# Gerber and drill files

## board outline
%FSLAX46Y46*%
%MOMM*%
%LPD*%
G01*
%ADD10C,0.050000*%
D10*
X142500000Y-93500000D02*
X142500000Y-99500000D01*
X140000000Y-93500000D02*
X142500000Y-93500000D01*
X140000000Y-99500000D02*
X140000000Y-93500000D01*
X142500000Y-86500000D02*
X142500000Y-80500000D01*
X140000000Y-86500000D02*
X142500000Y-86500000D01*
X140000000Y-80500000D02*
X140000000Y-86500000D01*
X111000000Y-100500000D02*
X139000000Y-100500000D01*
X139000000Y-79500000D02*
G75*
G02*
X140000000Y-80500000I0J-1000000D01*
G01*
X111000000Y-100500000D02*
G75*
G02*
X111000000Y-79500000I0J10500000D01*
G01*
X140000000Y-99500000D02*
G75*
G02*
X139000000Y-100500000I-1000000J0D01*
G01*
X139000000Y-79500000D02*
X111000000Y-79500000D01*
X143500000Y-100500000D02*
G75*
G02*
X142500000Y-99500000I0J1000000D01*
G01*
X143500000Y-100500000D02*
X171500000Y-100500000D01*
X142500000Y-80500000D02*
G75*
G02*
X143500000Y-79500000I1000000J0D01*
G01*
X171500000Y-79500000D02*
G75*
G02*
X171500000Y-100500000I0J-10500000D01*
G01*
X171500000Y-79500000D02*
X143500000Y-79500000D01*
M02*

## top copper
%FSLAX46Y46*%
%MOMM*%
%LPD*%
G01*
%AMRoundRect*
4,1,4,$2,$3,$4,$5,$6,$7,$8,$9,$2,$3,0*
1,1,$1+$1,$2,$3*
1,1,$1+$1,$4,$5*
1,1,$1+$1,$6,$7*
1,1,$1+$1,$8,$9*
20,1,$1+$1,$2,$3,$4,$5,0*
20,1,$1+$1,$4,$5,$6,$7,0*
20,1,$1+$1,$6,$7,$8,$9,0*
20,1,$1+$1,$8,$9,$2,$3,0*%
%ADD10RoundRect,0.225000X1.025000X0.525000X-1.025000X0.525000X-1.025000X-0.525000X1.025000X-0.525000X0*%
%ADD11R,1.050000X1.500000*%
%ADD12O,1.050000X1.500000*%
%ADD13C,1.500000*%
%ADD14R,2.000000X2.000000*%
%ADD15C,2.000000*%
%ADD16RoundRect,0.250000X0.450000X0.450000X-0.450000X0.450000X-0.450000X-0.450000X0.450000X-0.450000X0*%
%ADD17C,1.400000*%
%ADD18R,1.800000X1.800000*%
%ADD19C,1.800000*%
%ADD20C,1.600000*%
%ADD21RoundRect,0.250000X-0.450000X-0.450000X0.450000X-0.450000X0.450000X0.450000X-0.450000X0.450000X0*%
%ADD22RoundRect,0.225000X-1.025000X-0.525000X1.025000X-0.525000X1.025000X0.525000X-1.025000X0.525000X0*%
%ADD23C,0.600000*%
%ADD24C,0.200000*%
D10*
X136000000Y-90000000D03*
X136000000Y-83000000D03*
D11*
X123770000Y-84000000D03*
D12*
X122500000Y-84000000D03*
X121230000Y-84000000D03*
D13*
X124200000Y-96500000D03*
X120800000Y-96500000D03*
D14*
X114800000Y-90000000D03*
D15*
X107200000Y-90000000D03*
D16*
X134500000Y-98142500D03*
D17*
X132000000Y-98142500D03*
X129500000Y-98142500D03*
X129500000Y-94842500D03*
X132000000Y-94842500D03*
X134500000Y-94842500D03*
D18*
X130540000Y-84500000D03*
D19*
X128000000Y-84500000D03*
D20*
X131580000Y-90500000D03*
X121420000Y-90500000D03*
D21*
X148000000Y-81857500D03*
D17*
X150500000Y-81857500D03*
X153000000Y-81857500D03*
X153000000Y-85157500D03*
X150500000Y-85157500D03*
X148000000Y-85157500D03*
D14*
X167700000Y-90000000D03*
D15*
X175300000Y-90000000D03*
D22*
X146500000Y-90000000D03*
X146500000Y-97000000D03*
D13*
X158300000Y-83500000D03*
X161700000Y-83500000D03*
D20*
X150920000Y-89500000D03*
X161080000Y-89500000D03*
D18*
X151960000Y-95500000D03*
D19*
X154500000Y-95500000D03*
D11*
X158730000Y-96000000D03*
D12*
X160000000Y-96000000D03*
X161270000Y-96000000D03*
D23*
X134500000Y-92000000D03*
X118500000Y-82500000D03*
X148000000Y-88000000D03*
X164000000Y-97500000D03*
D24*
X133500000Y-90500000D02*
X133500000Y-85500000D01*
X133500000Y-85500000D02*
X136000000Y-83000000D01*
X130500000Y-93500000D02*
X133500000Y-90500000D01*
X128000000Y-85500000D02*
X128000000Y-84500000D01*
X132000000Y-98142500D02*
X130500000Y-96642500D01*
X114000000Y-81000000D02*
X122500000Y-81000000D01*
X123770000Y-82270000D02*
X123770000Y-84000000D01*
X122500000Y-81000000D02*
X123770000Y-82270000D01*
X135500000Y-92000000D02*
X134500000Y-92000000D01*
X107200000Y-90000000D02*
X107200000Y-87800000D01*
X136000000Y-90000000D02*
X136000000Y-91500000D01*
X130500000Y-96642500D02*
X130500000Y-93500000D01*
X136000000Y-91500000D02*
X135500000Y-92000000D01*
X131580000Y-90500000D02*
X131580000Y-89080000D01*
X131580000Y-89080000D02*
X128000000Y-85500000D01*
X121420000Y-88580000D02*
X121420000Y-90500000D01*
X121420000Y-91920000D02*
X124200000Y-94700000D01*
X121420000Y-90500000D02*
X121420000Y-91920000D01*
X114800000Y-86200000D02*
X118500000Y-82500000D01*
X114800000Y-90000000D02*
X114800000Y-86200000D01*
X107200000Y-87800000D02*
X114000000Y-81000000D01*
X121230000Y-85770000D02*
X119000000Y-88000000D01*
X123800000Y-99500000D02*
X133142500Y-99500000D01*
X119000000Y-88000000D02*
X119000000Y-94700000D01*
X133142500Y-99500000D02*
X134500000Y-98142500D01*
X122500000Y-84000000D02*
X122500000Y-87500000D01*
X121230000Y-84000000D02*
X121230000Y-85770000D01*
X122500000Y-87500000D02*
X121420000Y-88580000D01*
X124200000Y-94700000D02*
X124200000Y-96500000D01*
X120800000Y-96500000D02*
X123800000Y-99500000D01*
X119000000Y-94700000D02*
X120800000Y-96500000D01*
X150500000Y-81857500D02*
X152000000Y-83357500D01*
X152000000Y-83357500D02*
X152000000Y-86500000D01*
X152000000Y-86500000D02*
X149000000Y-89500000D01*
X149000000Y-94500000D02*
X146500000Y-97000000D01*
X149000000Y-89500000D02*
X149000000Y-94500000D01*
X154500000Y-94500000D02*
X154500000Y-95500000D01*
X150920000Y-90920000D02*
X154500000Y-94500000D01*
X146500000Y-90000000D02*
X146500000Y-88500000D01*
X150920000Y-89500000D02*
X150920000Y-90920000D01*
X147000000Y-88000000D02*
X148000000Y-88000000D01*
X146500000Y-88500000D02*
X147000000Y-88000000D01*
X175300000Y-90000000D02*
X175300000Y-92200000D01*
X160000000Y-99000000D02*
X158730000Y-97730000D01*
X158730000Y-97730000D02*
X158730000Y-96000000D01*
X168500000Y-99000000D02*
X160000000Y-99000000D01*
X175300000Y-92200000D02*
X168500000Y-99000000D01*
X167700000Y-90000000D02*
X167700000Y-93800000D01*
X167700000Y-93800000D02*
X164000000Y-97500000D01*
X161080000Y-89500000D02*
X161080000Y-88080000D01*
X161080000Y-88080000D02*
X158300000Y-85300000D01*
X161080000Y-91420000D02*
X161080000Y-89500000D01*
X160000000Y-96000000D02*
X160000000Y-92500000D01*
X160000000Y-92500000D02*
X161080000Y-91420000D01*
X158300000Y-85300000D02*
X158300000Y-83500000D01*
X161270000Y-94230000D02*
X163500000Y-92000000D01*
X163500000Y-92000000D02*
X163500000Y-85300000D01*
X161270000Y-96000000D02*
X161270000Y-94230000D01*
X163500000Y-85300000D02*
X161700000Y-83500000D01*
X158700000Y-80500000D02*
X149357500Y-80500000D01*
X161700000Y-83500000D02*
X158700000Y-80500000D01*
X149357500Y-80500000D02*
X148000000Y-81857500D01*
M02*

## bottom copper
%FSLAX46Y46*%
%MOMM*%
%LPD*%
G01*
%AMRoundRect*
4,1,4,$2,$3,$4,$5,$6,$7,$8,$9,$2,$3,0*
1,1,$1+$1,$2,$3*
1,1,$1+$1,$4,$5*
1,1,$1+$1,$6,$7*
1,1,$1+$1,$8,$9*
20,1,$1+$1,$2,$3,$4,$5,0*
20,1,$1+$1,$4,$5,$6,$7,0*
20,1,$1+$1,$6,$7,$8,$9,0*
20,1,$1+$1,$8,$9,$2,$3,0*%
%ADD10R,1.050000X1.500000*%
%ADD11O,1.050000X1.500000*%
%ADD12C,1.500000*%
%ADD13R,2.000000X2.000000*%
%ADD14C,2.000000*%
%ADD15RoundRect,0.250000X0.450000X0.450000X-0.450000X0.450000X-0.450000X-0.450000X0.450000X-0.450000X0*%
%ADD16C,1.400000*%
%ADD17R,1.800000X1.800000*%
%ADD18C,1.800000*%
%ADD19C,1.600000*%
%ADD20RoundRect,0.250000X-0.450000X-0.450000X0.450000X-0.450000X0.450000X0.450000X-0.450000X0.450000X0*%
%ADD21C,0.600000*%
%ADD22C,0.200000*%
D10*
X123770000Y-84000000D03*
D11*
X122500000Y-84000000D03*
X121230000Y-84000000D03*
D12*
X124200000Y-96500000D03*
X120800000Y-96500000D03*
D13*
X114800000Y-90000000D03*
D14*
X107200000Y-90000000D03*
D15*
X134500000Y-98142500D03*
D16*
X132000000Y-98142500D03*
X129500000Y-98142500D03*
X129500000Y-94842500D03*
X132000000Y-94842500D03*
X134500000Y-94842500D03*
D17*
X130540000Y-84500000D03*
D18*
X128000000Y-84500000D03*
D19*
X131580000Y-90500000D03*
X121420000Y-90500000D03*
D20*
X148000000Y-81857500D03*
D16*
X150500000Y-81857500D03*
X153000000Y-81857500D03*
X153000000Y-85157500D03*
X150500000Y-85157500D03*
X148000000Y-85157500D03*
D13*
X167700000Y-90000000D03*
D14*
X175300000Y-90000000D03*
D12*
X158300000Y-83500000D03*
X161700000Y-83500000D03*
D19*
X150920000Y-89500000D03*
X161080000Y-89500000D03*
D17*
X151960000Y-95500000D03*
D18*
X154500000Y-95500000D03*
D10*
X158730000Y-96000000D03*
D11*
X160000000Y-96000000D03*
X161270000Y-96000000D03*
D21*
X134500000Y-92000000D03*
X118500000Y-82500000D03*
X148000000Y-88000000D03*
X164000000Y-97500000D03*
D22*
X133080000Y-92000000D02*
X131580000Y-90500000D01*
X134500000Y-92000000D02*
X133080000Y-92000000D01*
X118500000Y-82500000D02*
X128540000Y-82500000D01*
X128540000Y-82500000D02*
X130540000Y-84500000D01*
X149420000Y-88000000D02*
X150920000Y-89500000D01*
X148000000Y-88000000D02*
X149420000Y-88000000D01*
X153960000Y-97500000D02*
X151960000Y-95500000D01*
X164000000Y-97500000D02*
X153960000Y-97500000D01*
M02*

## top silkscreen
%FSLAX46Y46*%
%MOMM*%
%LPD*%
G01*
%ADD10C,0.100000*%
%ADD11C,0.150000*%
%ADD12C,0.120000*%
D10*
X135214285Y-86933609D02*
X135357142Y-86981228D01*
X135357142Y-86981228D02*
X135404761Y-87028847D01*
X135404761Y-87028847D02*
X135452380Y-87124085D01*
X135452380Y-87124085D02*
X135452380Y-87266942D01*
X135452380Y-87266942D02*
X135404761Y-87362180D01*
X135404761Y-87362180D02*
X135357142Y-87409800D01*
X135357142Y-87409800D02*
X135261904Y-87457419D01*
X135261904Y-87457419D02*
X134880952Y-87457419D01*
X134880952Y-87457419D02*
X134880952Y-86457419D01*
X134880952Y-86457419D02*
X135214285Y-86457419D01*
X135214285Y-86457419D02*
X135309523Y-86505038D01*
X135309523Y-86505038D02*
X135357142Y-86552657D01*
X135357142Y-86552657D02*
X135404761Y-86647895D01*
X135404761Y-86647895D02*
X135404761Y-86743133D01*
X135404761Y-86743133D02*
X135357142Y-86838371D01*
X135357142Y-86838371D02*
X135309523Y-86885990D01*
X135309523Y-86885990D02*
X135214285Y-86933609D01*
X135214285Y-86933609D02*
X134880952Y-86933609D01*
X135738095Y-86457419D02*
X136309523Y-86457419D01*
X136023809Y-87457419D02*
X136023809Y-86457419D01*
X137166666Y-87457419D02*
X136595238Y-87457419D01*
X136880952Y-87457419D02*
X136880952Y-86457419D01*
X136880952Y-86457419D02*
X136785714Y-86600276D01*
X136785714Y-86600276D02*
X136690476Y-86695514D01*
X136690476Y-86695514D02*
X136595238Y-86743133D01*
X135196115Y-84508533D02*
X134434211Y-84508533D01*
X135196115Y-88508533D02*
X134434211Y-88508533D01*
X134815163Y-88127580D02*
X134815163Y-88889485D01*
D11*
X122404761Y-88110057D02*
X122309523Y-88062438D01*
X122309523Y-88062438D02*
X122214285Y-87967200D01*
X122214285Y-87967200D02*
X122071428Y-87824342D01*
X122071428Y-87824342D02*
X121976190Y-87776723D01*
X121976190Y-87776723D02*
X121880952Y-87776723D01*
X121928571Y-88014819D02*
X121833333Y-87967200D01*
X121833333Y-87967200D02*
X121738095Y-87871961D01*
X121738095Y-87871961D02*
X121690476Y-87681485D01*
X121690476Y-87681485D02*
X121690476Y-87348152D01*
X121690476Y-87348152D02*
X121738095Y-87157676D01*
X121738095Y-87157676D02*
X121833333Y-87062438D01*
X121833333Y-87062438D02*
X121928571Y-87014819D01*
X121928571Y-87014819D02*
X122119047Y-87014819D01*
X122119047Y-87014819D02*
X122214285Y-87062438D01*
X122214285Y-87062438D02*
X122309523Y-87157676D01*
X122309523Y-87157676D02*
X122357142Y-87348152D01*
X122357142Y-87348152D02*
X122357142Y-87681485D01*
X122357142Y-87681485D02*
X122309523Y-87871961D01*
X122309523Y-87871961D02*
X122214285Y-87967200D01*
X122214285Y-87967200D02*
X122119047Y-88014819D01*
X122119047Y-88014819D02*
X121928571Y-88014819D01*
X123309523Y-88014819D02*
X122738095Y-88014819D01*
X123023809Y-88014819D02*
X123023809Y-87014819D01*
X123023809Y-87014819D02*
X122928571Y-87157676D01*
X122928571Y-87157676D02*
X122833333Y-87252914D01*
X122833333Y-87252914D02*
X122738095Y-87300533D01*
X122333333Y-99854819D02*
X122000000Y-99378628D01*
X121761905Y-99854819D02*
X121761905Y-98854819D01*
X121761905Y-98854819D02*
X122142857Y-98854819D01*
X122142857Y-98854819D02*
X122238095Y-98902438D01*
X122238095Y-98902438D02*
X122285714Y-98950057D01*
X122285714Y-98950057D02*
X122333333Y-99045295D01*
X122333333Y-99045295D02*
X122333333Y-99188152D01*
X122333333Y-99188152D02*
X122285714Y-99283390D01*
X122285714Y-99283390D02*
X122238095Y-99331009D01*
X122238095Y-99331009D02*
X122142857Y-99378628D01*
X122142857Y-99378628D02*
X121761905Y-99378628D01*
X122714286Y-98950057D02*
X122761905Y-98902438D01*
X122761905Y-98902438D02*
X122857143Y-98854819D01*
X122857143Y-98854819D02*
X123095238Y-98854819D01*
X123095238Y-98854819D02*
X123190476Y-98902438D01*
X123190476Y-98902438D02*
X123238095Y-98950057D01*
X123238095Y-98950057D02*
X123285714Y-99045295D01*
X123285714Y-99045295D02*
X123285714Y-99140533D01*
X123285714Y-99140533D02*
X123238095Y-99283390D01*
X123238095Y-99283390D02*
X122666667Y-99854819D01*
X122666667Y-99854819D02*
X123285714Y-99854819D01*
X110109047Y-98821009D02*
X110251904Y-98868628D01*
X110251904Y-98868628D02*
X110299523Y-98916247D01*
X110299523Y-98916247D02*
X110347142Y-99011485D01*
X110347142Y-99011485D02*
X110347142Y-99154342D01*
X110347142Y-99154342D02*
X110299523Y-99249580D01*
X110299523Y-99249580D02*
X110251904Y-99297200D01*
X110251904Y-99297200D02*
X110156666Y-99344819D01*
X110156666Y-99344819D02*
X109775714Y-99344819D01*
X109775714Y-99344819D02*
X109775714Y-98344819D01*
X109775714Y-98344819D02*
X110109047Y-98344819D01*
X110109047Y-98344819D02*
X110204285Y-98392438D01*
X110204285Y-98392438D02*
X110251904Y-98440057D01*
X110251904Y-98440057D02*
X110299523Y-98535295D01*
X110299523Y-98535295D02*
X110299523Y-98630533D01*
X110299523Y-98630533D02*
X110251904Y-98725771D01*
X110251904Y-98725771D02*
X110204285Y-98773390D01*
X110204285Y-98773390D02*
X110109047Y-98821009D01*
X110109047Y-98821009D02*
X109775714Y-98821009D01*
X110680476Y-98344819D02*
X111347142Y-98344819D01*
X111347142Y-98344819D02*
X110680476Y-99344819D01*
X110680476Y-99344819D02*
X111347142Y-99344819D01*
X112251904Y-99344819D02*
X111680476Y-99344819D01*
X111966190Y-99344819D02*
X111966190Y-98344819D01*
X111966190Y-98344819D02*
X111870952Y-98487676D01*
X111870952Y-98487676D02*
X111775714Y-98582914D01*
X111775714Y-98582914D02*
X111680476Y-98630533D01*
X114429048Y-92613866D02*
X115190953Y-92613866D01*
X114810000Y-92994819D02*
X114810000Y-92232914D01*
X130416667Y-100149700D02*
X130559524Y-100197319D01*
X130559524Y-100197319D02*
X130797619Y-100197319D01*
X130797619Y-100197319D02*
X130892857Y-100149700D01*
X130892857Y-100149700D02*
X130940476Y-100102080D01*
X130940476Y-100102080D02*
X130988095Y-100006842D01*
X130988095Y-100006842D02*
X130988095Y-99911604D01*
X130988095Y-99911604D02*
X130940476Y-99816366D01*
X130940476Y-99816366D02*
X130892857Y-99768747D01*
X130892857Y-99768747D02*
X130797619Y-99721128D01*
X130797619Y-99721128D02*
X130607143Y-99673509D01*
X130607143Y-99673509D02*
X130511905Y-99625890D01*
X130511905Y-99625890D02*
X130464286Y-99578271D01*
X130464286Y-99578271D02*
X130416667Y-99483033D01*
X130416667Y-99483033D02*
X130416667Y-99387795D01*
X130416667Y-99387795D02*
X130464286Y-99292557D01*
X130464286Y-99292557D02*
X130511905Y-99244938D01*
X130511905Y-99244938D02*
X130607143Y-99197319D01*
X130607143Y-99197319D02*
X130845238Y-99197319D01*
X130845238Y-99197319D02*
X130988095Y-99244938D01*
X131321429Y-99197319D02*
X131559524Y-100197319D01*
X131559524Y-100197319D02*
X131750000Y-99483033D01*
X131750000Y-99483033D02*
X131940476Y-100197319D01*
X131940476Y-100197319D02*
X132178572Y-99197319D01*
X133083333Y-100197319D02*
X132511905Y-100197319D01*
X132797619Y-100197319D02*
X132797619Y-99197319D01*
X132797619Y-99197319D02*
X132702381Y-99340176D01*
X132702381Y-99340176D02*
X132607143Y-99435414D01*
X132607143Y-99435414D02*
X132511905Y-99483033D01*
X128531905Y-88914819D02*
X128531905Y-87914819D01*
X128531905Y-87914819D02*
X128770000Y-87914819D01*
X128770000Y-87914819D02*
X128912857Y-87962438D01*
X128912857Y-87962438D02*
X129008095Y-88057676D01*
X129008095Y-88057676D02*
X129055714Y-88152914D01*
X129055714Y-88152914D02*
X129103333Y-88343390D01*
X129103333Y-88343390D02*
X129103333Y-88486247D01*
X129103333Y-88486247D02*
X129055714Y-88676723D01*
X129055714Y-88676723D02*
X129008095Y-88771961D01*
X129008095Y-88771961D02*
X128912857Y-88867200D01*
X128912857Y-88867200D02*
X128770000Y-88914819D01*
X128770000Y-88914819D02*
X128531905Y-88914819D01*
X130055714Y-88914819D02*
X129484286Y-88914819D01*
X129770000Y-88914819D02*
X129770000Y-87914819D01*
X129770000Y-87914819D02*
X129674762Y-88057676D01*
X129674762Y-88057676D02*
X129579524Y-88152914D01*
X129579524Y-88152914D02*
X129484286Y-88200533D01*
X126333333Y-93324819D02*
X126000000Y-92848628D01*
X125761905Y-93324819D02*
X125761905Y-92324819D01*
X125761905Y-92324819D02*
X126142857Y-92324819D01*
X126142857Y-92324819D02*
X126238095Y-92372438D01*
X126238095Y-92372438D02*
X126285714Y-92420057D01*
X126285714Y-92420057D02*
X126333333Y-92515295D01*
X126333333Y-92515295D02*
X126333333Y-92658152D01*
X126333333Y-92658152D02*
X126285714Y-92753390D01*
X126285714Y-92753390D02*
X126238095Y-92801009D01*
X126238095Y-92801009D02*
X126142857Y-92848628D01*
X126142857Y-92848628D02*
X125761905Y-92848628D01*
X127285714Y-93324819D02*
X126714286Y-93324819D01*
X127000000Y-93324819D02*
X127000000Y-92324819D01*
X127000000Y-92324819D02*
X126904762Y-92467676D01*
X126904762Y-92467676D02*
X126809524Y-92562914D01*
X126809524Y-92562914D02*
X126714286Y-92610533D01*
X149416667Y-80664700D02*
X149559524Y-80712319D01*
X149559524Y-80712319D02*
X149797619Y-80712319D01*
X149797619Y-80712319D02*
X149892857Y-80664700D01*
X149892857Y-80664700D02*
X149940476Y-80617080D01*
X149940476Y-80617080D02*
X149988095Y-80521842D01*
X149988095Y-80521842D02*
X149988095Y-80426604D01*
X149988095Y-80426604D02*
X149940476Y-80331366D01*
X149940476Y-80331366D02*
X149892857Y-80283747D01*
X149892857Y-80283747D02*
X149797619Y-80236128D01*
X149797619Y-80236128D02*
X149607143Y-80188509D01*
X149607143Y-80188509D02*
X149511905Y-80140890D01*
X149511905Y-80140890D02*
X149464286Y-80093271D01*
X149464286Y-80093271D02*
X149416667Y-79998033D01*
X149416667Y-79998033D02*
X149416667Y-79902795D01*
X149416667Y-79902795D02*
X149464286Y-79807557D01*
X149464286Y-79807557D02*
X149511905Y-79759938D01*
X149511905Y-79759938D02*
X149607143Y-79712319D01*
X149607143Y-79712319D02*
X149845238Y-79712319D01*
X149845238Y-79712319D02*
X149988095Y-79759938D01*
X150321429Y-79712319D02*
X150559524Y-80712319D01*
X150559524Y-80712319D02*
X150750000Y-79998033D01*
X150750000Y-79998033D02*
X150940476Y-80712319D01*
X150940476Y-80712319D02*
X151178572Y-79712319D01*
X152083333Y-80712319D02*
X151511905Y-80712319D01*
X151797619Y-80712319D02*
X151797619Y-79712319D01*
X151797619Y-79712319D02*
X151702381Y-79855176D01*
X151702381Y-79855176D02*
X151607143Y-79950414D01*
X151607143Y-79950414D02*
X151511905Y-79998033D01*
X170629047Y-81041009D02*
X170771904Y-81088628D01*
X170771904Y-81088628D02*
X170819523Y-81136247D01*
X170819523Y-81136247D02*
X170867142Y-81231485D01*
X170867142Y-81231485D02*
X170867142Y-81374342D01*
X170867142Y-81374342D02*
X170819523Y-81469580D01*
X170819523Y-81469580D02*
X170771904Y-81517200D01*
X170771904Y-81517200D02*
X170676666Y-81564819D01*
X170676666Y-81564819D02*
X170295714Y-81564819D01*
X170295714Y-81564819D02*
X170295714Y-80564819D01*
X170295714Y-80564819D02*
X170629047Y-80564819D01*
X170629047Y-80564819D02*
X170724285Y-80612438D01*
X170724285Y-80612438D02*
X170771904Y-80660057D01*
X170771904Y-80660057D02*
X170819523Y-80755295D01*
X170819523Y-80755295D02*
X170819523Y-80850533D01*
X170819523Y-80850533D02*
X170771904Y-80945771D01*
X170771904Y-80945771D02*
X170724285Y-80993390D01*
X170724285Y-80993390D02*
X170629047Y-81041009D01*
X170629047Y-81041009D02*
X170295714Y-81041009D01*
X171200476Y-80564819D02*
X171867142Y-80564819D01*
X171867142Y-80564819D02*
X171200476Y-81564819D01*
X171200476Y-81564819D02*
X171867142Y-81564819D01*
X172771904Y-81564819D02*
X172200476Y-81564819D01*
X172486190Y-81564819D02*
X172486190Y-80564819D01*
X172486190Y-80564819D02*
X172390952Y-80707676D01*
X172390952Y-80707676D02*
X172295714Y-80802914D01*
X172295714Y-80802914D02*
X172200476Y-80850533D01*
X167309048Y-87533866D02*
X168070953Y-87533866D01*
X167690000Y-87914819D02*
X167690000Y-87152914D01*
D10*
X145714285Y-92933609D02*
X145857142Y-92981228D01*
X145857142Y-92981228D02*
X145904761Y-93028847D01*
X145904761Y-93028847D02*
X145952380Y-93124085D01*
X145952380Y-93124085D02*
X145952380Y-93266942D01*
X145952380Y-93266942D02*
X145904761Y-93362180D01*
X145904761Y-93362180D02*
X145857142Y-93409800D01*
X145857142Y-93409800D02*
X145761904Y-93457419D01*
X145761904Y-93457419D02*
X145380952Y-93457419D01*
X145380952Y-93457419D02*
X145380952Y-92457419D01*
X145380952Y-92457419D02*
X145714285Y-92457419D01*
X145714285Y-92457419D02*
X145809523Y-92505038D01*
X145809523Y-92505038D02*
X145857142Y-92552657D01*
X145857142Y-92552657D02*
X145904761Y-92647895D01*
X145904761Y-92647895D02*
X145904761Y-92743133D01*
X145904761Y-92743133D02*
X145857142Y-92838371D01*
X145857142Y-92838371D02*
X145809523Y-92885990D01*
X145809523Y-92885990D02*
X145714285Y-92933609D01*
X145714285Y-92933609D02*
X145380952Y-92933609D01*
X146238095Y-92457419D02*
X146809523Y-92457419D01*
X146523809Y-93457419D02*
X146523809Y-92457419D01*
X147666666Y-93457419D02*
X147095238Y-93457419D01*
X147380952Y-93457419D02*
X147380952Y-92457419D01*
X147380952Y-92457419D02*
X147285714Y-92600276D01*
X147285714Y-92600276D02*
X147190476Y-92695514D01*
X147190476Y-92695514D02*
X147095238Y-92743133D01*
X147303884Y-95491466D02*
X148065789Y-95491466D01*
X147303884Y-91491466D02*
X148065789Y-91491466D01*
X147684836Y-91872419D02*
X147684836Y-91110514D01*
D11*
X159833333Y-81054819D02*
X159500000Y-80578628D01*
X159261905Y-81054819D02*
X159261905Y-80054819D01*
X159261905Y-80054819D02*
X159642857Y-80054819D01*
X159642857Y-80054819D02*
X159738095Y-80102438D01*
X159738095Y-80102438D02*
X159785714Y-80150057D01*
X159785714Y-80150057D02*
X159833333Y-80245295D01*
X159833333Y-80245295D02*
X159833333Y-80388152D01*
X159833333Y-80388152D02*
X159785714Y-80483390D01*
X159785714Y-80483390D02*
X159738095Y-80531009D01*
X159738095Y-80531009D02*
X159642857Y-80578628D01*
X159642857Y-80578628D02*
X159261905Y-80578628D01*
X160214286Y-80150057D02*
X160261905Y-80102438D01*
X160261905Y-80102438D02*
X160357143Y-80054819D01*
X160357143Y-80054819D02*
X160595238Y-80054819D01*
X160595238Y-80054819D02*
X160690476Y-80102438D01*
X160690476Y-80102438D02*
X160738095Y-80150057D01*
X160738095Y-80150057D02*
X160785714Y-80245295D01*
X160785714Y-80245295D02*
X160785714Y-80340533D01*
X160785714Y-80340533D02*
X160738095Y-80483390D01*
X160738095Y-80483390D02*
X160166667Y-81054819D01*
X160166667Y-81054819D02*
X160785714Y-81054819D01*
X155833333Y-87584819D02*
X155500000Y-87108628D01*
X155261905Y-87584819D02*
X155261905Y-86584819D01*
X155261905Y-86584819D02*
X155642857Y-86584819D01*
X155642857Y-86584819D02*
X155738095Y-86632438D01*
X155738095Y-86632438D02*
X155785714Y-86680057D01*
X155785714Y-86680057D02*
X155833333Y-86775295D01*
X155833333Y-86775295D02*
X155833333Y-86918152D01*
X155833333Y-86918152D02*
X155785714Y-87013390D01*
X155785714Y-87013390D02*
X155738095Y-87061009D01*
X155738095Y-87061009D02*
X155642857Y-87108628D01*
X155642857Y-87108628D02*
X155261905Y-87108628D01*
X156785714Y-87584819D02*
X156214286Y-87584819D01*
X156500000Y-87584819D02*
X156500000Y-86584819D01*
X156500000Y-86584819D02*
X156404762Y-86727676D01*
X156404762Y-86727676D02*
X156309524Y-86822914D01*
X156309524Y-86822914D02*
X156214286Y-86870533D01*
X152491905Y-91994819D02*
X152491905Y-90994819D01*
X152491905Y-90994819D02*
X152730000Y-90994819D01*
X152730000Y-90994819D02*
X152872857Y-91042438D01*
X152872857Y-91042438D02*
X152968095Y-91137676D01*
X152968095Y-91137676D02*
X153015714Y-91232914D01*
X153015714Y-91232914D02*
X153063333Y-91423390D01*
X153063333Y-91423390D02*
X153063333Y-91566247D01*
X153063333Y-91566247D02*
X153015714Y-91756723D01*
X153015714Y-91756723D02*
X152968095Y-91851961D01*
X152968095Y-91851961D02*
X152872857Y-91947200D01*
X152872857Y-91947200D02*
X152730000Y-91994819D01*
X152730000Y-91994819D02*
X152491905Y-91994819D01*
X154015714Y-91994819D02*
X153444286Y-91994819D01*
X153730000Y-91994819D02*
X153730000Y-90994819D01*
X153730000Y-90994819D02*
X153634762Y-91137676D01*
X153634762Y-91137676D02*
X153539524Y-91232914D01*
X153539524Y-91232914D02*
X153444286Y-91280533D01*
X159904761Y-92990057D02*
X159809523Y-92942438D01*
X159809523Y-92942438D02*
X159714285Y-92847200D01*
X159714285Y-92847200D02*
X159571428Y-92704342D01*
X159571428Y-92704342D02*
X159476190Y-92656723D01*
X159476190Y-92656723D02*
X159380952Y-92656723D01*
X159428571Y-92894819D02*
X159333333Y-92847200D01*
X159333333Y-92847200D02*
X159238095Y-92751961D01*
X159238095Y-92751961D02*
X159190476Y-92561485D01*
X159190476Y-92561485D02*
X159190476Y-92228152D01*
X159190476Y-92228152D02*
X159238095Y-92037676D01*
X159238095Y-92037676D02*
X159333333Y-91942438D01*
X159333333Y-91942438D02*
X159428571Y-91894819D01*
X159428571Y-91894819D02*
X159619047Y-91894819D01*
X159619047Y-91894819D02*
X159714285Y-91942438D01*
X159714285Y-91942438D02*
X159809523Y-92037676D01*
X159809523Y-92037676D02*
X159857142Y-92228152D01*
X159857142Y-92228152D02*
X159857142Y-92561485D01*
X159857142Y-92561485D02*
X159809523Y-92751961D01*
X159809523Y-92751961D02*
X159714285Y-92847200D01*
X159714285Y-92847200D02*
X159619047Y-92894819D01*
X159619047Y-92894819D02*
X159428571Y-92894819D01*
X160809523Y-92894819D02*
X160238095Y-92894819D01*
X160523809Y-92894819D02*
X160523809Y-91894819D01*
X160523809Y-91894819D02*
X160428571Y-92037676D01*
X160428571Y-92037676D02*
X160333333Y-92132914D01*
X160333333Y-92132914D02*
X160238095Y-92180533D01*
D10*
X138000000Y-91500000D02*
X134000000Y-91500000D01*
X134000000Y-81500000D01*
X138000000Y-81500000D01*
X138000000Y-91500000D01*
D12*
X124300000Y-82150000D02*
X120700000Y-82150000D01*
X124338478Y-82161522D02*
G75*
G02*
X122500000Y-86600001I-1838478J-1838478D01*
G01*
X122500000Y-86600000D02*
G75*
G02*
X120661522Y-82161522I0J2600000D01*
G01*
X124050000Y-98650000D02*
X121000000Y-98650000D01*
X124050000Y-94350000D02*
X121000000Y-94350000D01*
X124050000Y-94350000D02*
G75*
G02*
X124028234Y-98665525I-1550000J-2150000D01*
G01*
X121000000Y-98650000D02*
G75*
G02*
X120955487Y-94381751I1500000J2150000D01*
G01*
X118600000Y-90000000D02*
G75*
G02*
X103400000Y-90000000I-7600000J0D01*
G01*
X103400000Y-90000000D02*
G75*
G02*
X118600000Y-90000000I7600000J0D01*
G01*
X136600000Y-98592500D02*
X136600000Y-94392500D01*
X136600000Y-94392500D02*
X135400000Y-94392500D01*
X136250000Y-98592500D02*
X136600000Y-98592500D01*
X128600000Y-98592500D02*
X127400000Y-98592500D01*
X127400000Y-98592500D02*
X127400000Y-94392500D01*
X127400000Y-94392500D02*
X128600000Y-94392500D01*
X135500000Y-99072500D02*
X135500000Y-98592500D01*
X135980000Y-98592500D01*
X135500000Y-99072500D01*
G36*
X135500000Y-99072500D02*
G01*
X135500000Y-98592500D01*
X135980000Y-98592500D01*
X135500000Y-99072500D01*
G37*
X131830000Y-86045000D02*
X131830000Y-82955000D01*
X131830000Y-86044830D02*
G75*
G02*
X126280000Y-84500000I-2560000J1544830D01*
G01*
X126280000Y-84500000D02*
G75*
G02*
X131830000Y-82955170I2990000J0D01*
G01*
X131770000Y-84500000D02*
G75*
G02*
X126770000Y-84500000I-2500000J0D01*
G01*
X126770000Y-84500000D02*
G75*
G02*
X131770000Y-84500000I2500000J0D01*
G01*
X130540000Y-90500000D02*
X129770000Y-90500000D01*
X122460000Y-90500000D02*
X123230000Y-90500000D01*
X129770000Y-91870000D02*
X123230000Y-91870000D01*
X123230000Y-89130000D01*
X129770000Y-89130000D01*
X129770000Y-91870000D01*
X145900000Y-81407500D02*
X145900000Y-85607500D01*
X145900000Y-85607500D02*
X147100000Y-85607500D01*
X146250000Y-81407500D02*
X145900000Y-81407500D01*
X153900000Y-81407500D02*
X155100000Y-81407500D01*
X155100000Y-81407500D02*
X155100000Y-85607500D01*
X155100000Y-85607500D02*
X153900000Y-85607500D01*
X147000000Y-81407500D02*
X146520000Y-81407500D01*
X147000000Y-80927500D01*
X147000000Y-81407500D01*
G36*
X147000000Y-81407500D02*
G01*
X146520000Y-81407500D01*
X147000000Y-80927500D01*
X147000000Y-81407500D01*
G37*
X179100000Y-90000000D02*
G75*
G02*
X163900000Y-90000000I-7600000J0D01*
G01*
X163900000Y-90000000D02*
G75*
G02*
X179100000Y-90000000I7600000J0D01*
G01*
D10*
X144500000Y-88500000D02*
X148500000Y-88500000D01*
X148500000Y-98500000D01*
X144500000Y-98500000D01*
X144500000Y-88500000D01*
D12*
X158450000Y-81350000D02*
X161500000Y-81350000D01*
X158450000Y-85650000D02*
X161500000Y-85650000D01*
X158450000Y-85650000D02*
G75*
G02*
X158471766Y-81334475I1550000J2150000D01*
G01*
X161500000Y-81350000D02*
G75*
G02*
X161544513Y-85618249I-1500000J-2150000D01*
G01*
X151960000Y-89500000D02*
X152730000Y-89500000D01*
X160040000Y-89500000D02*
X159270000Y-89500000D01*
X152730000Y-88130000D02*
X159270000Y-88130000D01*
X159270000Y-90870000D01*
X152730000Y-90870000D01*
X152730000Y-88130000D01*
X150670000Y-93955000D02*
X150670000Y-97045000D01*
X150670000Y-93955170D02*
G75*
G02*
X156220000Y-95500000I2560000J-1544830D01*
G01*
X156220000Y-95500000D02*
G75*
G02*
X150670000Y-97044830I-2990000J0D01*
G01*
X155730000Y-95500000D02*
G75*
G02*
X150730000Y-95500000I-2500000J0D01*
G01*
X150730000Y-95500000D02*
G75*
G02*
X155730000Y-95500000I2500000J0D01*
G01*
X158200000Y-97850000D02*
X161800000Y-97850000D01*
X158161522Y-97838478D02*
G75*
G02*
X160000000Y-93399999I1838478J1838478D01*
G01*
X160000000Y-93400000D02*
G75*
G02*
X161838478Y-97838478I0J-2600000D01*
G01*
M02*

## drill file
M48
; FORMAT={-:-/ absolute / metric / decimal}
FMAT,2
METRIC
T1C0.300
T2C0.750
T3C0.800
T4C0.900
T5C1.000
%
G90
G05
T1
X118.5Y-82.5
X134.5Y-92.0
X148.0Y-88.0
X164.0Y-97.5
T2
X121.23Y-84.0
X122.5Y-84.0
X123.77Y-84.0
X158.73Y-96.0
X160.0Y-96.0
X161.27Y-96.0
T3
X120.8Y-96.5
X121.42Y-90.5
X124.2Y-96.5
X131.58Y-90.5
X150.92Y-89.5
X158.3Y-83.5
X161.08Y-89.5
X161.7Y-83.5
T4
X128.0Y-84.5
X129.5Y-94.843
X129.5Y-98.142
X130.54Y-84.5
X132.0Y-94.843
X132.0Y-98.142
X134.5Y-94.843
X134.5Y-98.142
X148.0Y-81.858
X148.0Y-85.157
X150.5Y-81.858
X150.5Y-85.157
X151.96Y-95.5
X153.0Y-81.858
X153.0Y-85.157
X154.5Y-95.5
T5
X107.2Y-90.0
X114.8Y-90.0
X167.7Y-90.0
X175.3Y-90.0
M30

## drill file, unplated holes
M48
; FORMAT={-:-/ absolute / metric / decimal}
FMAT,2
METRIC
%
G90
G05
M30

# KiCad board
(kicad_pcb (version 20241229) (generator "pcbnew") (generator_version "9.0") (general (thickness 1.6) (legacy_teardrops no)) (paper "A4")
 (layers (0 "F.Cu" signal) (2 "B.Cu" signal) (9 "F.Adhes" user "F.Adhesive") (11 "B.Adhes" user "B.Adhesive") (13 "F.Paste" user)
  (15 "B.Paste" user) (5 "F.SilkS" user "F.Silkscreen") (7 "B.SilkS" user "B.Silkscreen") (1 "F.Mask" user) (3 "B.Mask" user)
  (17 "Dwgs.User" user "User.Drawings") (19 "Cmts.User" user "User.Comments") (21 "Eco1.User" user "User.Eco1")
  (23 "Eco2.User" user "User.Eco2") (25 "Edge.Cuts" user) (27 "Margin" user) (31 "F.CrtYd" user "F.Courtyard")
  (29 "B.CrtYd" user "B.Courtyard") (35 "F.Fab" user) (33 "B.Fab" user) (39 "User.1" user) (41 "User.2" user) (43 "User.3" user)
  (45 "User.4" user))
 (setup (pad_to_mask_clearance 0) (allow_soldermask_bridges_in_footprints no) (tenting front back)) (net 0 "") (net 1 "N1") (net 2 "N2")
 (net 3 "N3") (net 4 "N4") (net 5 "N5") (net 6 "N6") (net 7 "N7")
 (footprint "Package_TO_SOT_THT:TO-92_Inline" (layer "F.Cu") (at 123.77 84 180)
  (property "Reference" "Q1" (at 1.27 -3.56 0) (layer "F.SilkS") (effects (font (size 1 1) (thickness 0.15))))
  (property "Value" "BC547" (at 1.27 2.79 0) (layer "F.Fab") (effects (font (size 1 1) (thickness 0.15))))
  (fp_line (start -0.53 1.85) (end 3.07 1.85) (stroke (width 0.12) (type solid)) (layer "F.SilkS"))
  (fp_arc (start 1.27 -2.6) (mid 3.672087 -0.994977) (end 3.108478 1.838478) (stroke (width 0.12) (type solid)) (layer "F.SilkS"))
  (fp_arc (start -0.568478 1.838478) (mid -1.132087 -0.994977) (end 1.27 -2.6) (stroke (width 0.12) (type solid)) (layer "F.SilkS"))
  (pad "1" thru_hole rect (at 0 0 180) (size 1.05 1.5) (drill 0.75) (layers "*.Cu" "*.Mask") (remove_unused_layers no) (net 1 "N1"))
  (pad "2" thru_hole oval (at 1.27 0 180) (size 1.05 1.5) (drill 0.75) (layers "*.Cu" "*.Mask") (remove_unused_layers no) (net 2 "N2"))
  (pad "3" thru_hole oval (at 2.54 0 180) (size 1.05 1.5) (drill 0.75) (layers "*.Cu" "*.Mask") (remove_unused_layers no) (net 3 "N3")))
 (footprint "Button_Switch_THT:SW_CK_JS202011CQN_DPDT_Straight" (layer "F.Cu") (at 148 81.8575)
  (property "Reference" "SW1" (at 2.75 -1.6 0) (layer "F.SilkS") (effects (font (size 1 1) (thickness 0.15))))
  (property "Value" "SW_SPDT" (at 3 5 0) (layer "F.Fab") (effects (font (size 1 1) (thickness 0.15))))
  (fp_line (start -2.1 -0.45) (end -2.1 3.75) (stroke (width 0.12) (type solid)) (layer "F.SilkS"))
  (fp_line (start -2.1 3.75) (end -0.9 3.75) (stroke (width 0.12) (type solid)) (layer "F.SilkS"))
  (fp_line (start -1.75 -0.45) (end -2.1 -0.45) (stroke (width 0.12) (type solid)) (layer "F.SilkS"))
  (fp_line (start 5.9 -0.45) (end 7.1 -0.45) (stroke (width 0.12) (type solid)) (layer "F.SilkS"))
  (fp_line (start 7.1 -0.45) (end 7.1 3.75) (stroke (width 0.12) (type solid)) (layer "F.SilkS"))
  (fp_line (start 7.1 3.75) (end 5.9 3.75) (stroke (width 0.12) (type solid)) (layer "F.SilkS"))
  (fp_poly (pts (xy -1 -0.45) (xy -1.48 -0.45) (xy -1 -0.93) (xy -1 -0.45)) (stroke (width 0.12) (type solid)) (fill yes) (layer "F.SilkS"))
  (pad "1" thru_hole roundrect (at 0 0) (size 1.4 1.4) (drill 0.9) (layers "*.Cu" "*.Mask") (remove_unused_layers no)
   (roundrect_rratio 0.1785714286) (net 3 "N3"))
  (pad "2" thru_hole circle (at 2.5 0) (size 1.4 1.4) (drill 0.9) (layers "*.Cu" "*.Mask") (remove_unused_layers no) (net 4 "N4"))
  (pad "3" thru_hole circle (at 5 0) (size 1.4 1.4) (drill 0.9) (layers "*.Cu" "*.Mask") (remove_unused_layers no) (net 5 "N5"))
  (pad "4" thru_hole circle (at 5 3.3) (size 1.4 1.4) (drill 0.9) (layers "*.Cu" "*.Mask") (remove_unused_layers no))
  (pad "5" thru_hole circle (at 2.5 3.3) (size 1.4 1.4) (drill 0.9) (layers "*.Cu" "*.Mask") (remove_unused_layers no))
  (pad "6" thru_hole circle (at 0 3.3) (size 1.4 1.4) (drill 0.9) (layers "*.Cu" "*.Mask") (remove_unused_layers no)))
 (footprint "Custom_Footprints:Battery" (layer "F.Cu") (at 136 86.5 180)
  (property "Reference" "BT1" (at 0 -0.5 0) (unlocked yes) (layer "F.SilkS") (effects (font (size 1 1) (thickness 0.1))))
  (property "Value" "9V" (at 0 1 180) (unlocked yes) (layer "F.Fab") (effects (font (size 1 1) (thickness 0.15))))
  (fp_rect (start -2 -5) (end 2 5) (stroke (width 0.1) (type default)) (fill no) (layer "F.SilkS"))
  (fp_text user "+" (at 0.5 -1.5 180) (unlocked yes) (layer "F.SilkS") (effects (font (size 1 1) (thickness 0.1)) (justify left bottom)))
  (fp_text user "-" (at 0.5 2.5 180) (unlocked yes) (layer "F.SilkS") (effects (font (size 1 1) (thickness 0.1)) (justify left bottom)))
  (pad "1" smd roundrect (at 0 -3.5 180) (size 2.5 1.5) (layers "F.Cu" "F.Mask" "F.Paste") (roundrect_rratio 0.15) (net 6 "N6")
   (thermal_bridge_angle 45))
  (pad "2" smd roundrect (at 0 3.5 180) (size 2.5 1.5) (layers "F.Cu" "F.Mask" "F.Paste") (roundrect_rratio 0.15) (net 4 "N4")
   (thermal_bridge_angle 45)))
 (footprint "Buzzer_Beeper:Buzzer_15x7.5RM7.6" (layer "F.Cu") (at 167.7 90)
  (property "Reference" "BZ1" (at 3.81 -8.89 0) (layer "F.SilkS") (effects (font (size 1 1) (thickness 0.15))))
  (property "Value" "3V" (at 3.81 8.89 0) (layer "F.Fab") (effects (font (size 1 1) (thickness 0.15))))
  (fp_circle (center 3.8 0) (end 11.4 0) (stroke (width 0.12) (type solid)) (fill no) (layer "F.SilkS"))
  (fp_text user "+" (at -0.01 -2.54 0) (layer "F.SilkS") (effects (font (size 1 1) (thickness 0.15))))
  (pad "1" thru_hole rect (at 0 0) (size 2 2) (drill 1) (layers "*.Cu" "*.Mask") (remove_unused_layers no) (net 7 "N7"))
  (pad "2" thru_hole circle (at 7.6 0) (size 2 2) (drill 1) (layers "*.Cu" "*.Mask") (remove_unused_layers no) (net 1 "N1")))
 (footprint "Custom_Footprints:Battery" (layer "F.Cu") (at 146.5 93.5)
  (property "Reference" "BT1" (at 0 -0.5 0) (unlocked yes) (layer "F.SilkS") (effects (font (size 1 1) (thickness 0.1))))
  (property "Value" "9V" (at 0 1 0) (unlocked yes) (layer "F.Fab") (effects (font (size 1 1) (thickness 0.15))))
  (fp_rect (start -2 -5) (end 2 5) (stroke (width 0.1) (type default)) (fill no) (layer "F.SilkS"))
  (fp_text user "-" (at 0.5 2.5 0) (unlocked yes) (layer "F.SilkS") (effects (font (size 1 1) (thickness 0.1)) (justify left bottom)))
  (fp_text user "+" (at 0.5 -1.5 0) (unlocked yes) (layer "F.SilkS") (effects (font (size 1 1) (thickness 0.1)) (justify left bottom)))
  (pad "1" smd roundrect (at 0 -3.5) (size 2.5 1.5) (layers "F.Cu" "F.Mask" "F.Paste") (roundrect_rratio 0.15) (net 6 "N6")
   (thermal_bridge_angle 45))
  (pad "2" smd roundrect (at 0 3.5) (size 2.5 1.5) (layers "F.Cu" "F.Mask" "F.Paste") (roundrect_rratio 0.15) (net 4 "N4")
   (thermal_bridge_angle 45)))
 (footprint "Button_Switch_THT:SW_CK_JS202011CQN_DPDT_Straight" (layer "F.Cu") (at 134.5 98.1425 180)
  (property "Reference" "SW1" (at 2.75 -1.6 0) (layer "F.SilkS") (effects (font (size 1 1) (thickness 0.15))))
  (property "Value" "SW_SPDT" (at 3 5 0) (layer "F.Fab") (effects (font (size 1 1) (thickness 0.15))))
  (fp_line (start 7.1 3.75) (end 5.9 3.75) (stroke (width 0.12) (type solid)) (layer "F.SilkS"))
  (fp_line (start 7.1 -0.45) (end 7.1 3.75) (stroke (width 0.12) (type solid)) (layer "F.SilkS"))
  (fp_line (start 5.9 -0.45) (end 7.1 -0.45) (stroke (width 0.12) (type solid)) (layer "F.SilkS"))
  (fp_line (start -1.75 -0.45) (end -2.1 -0.45) (stroke (width 0.12) (type solid)) (layer "F.SilkS"))
  (fp_line (start -2.1 3.75) (end -0.9 3.75) (stroke (width 0.12) (type solid)) (layer "F.SilkS"))
  (fp_line (start -2.1 -0.45) (end -2.1 3.75) (stroke (width 0.12) (type solid)) (layer "F.SilkS"))
  (fp_poly (pts (xy -1 -0.45) (xy -1.48 -0.45) (xy -1 -0.93) (xy -1 -0.45)) (stroke (width 0.12) (type solid)) (fill yes) (layer "F.SilkS"))
  (pad "1" thru_hole roundrect (at 0 0 180) (size 1.4 1.4) (drill 0.9) (layers "*.Cu" "*.Mask") (remove_unused_layers no)
   (roundrect_rratio 0.1785714286) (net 3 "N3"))
  (pad "2" thru_hole circle (at 2.5 0 180) (size 1.4 1.4) (drill 0.9) (layers "*.Cu" "*.Mask") (remove_unused_layers no) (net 4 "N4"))
  (pad "3" thru_hole circle (at 5 0 180) (size 1.4 1.4) (drill 0.9) (layers "*.Cu" "*.Mask") (remove_unused_layers no) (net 5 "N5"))
  (pad "4" thru_hole circle (at 5 3.3 180) (size 1.4 1.4) (drill 0.9) (layers "*.Cu" "*.Mask") (remove_unused_layers no))
  (pad "5" thru_hole circle (at 2.5 3.3 180) (size 1.4 1.4) (drill 0.9) (layers "*.Cu" "*.Mask") (remove_unused_layers no))
  (pad "6" thru_hole circle (at 0 3.3 180) (size 1.4 1.4) (drill 0.9) (layers "*.Cu" "*.Mask") (remove_unused_layers no)))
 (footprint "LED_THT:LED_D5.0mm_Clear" (layer "F.Cu") (at 130.54 84.5 180)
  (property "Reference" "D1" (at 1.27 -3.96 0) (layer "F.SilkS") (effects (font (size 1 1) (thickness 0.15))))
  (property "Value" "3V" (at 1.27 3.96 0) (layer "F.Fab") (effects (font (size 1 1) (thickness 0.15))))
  (fp_line (start -1.29 -1.545) (end -1.29 1.545) (stroke (width 0.12) (type solid)) (layer "F.SilkS"))
  (fp_arc (start 4.26 0) (mid 2.071779 2.880495) (end -1.29 1.54483) (stroke (width 0.12) (type solid)) (layer "F.SilkS"))
  (fp_arc (start -1.29 -1.54483) (mid 2.071779 -2.880495) (end 4.26 0) (stroke (width 0.12) (type solid)) (layer "F.SilkS"))
  (fp_circle (center 1.27 0) (end 3.77 0) (stroke (width 0.12) (type solid)) (fill no) (layer "F.SilkS"))
  (pad "1" thru_hole rect (at 0 0 180) (size 1.8 1.8) (drill 0.9) (layers "*.Cu" "*.Mask") (remove_unused_layers no) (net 7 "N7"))
  (pad "2" thru_hole circle (at 2.54 0 180) (size 1.8 1.8) (drill 0.9) (layers "*.Cu" "*.Mask") (remove_unused_layers no) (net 6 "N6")))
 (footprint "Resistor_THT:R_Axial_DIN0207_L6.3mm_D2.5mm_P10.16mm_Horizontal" (layer "F.Cu") (at 131.58 90.5 180)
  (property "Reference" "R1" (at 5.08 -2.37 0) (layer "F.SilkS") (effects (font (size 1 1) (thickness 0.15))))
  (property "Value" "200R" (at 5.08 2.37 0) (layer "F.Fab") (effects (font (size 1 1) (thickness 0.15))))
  (fp_line (start 9.12 0) (end 8.35 0) (stroke (width 0.12) (type solid)) (layer "F.SilkS"))
  (fp_line (start 1.04 0) (end 1.81 0) (stroke (width 0.12) (type solid)) (layer "F.SilkS"))
  (fp_rect (start 1.81 -1.37) (end 8.35 1.37) (stroke (width 0.12) (type solid)) (fill no) (layer "F.SilkS"))
  (pad "1" thru_hole circle (at 0 0 180) (size 1.6 1.6) (drill 0.8) (layers "*.Cu" "*.Mask") (remove_unused_layers no) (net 6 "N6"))
  (pad "2" thru_hole circle (at 10.16 0 180) (size 1.6 1.6) (drill 0.8) (layers "*.Cu" "*.Mask") (remove_unused_layers no) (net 2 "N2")))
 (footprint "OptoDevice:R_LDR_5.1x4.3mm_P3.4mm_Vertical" (layer "F.Cu") (at 158.3 83.5)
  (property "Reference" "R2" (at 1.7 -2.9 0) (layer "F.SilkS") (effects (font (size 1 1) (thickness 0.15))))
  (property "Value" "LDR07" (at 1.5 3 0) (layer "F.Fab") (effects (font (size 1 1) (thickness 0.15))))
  (fp_line (start 0.15 -2.15) (end 3.2 -2.15) (stroke (width 0.12) (type solid)) (layer "F.SilkS"))
  (fp_line (start 0.15 2.15) (end 3.2 2.15) (stroke (width 0.12) (type solid)) (layer "F.SilkS"))
  (fp_arc (start 0.15 2.15) (mid -0.950438 -0.013368) (end 0.171766 -2.165525) (stroke (width 0.12) (type solid)) (layer "F.SilkS"))
  (fp_arc (start 3.2 -2.15) (mid 4.321403 -0.027338) (end 3.244513 2.118249) (stroke (width 0.12) (type solid)) (layer "F.SilkS"))
  (pad "1" thru_hole circle (at 0 0) (size 1.5 1.5) (drill 0.8) (layers "*.Cu" "*.Mask") (remove_unused_layers no) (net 2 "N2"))
  (pad "2" thru_hole circle (at 3.4 0) (size 1.5 1.5) (drill 0.8) (layers "*.Cu" "*.Mask") (remove_unused_layers no) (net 3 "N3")))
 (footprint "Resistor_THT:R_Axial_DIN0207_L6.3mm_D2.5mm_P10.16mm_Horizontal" (layer "F.Cu") (at 150.92 89.5)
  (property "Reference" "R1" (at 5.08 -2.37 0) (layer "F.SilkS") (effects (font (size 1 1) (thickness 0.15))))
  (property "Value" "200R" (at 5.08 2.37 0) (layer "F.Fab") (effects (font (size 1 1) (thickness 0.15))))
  (fp_line (start 1.04 0) (end 1.81 0) (stroke (width 0.12) (type solid)) (layer "F.SilkS"))
  (fp_line (start 9.12 0) (end 8.35 0) (stroke (width 0.12) (type solid)) (layer "F.SilkS"))
  (fp_rect (start 1.81 -1.37) (end 8.35 1.37) (stroke (width 0.12) (type solid)) (fill no) (layer "F.SilkS"))
  (pad "1" thru_hole circle (at 0 0) (size 1.6 1.6) (drill 0.8) (layers "*.Cu" "*.Mask") (remove_unused_layers no) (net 6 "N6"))
  (pad "2" thru_hole circle (at 10.16 0) (size 1.6 1.6) (drill 0.8) (layers "*.Cu" "*.Mask") (remove_unused_layers no) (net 2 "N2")))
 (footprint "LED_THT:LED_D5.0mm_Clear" (layer "F.Cu") (at 151.96 95.5)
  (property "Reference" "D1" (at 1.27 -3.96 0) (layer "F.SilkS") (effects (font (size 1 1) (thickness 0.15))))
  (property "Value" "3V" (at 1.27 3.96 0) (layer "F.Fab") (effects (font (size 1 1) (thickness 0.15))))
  (fp_line (start -1.29 -1.545) (end -1.29 1.545) (stroke (width 0.12) (type solid)) (layer "F.SilkS"))
  (fp_arc (start -1.29 -1.54483) (mid 2.071779 -2.880495) (end 4.26 0) (stroke (width 0.12) (type solid)) (layer "F.SilkS"))
  (fp_arc (start 4.26 0) (mid 2.071779 2.880495) (end -1.29 1.54483) (stroke (width 0.12) (type solid)) (layer "F.SilkS"))
  (fp_circle (center 1.27 0) (end 3.77 0) (stroke (width 0.12) (type solid)) (fill no) (layer "F.SilkS"))
  (pad "1" thru_hole rect (at 0 0) (size 1.8 1.8) (drill 0.9) (layers "*.Cu" "*.Mask") (remove_unused_layers no) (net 7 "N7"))
  (pad "2" thru_hole circle (at 2.54 0) (size 1.8 1.8) (drill 0.9) (layers "*.Cu" "*.Mask") (remove_unused_layers no) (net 6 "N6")))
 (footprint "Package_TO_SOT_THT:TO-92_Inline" (layer "F.Cu") (at 158.73 96)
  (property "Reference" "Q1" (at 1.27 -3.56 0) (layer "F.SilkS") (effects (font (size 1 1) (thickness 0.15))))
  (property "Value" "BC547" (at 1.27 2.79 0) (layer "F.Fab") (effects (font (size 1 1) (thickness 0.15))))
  (fp_line (start -0.53 1.85) (end 3.07 1.85) (stroke (width 0.12) (type solid)) (layer "F.SilkS"))
  (fp_arc (start -0.568478 1.838478) (mid -1.132087 -0.994977) (end 1.27 -2.6) (stroke (width 0.12) (type solid)) (layer "F.SilkS"))
  (fp_arc (start 1.27 -2.6) (mid 3.672087 -0.994977) (end 3.108478 1.838478) (stroke (width 0.12) (type solid)) (layer "F.SilkS"))
  (pad "1" thru_hole rect (at 0 0) (size 1.05 1.5) (drill 0.75) (layers "*.Cu" "*.Mask") (remove_unused_layers no) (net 1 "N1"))
  (pad "2" thru_hole oval (at 1.27 0) (size 1.05 1.5) (drill 0.75) (layers "*.Cu" "*.Mask") (remove_unused_layers no) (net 2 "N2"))
  (pad "3" thru_hole oval (at 2.54 0) (size 1.05 1.5) (drill 0.75) (layers "*.Cu" "*.Mask") (remove_unused_layers no) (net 3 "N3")))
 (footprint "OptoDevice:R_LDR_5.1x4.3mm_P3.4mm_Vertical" (layer "F.Cu") (at 124.2 96.5 180)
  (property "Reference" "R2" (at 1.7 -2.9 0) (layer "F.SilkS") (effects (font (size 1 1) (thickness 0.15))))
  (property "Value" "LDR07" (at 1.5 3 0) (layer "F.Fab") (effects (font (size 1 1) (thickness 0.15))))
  (fp_line (start 0.15 2.15) (end 3.2 2.15) (stroke (width 0.12) (type solid)) (layer "F.SilkS"))
  (fp_line (start 0.15 -2.15) (end 3.2 -2.15) (stroke (width 0.12) (type solid)) (layer "F.SilkS"))
  (fp_arc (start 3.2 -2.15) (mid 4.321403 -0.027338) (end 3.244513 2.118249) (stroke (width 0.12) (type solid)) (layer "F.SilkS"))
  (fp_arc (start 0.15 2.15) (mid -0.950438 -0.013368) (end 0.171766 -2.165525) (stroke (width 0.12) (type solid)) (layer "F.SilkS"))
  (pad "1" thru_hole circle (at 0 0 180) (size 1.5 1.5) (drill 0.8) (layers "*.Cu" "*.Mask") (remove_unused_layers no) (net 2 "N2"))
  (pad "2" thru_hole circle (at 3.4 0 180) (size 1.5 1.5) (drill 0.8) (layers "*.Cu" "*.Mask") (remove_unused_layers no) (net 3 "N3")))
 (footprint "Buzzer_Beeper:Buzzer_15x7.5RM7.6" (layer "F.Cu") (at 114.8 90 180)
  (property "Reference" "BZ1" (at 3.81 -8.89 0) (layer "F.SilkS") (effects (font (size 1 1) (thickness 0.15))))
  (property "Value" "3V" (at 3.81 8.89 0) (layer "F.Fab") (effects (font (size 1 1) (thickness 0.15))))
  (fp_circle (center 3.8 0) (end 11.4 0) (stroke (width 0.12) (type solid)) (fill no) (layer "F.SilkS"))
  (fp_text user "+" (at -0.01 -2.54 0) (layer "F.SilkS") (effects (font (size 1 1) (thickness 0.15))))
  (pad "1" thru_hole rect (at 0 0 180) (size 2 2) (drill 1) (layers "*.Cu" "*.Mask") (remove_unused_layers no) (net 7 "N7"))
  (pad "2" thru_hole circle (at 7.6 0 180) (size 2 2) (drill 1) (layers "*.Cu" "*.Mask") (remove_unused_layers no) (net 1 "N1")))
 (gr_arc (start 143.5 100.5) (mid 142.792893 100.207107) (end 142.5 99.5) (stroke (width 0.05) (type default)) (layer "Edge.Cuts"))
 (gr_line (start 111 100.5) (end 139 100.5) (stroke (width 0.05) (type default)) (layer "Edge.Cuts"))
 (gr_line (start 139 79.5) (end 111 79.5) (stroke (width 0.05) (type default)) (layer "Edge.Cuts"))
 (gr_arc (start 139 79.5) (mid 139.707107 79.792893) (end 140 80.5) (stroke (width 0.05) (type default)) (layer "Edge.Cuts"))
 (gr_line (start 140 93.5) (end 142.5 93.5) (stroke (width 0.05) (type default)) (layer "Edge.Cuts"))
 (gr_arc (start 111 100.5) (mid 100.5 90) (end 111 79.5) (stroke (width 0.05) (type default)) (layer "Edge.Cuts"))
 (gr_line (start 142.5 86.5) (end 142.5 80.5) (stroke (width 0.05) (type default)) (layer "Edge.Cuts"))
 (gr_line (start 143.5 100.5) (end 171.5 100.5) (stroke (width 0.05) (type default)) (layer "Edge.Cuts"))
 (gr_arc (start 142.5 80.5) (mid 142.792893 79.792893) (end 143.5 79.5) (stroke (width 0.05) (type default)) (layer "Edge.Cuts"))
 (gr_arc (start 171.5 79.5) (mid 182 90) (end 171.5 100.5) (stroke (width 0.05) (type default)) (layer "Edge.Cuts"))
 (gr_line (start 140 99.5) (end 140 93.5) (stroke (width 0.05) (type default)) (layer "Edge.Cuts"))
 (gr_line (start 140 80.5) (end 140 86.5) (stroke (width 0.05) (type default)) (layer "Edge.Cuts"))
 (gr_line (start 142.5 93.5) (end 142.5 99.5) (stroke (width 0.05) (type default)) (layer "Edge.Cuts"))
 (gr_arc (start 140 99.5) (mid 139.707107 100.207107) (end 139 100.5) (stroke (width 0.05) (type default)) (layer "Edge.Cuts"))
 (gr_line (start 140 86.5) (end 142.5 86.5) (stroke (width 0.05) (type default)) (layer "Edge.Cuts"))
 (gr_line (start 171.5 79.5) (end 143.5 79.5) (stroke (width 0.05) (type default)) (layer "Edge.Cuts"))
 (segment (start 133.5 85.5) (end 136 83) (width 0.2) (layer "F.Cu") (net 4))
 (segment (start 133.5 90.5) (end 133.5 85.5) (width 0.2) (layer "F.Cu") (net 4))
 (segment (start 150.5 81.8575) (end 152 83.3575) (width 0.2) (layer "F.Cu") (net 4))
 (segment (start 152 83.3575) (end 152 86.5) (width 0.2) (layer "F.Cu") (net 4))
 (segment (start 152 86.5) (end 149 89.5) (width 0.2) (layer "F.Cu") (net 4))
 (segment (start 130.5 93.5) (end 133.5 90.5) (width 0.2) (layer "F.Cu") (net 4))
 (segment (start 149 94.5) (end 146.5 97) (width 0.2) (layer "F.Cu") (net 4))
 (segment (start 132 98.1425) (end 130.5 96.6425) (width 0.2) (layer "F.Cu") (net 4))
 (segment (start 149 89.5) (end 149 94.5) (width 0.2) (layer "F.Cu") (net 4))
 (segment (start 130.5 96.6425) (end 130.5 93.5) (width 0.2) (layer "F.Cu") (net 4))
 (segment (start 154.5 94.5) (end 154.5 95.5) (width 0.2) (layer "F.Cu") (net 6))
 (segment (start 136 90) (end 136 91.5) (width 0.2) (layer "F.Cu") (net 6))
 (segment (start 150.92 90.92) (end 154.5 94.5) (width 0.2) (layer "F.Cu") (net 6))
 (segment (start 136 91.5) (end 135.5 92) (width 0.2) (layer "F.Cu") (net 6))
 (segment (start 146.5 90) (end 146.5 88.5) (width 0.2) (layer "F.Cu") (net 6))
 (segment (start 150.92 89.5) (end 150.92 90.92) (width 0.2) (layer "F.Cu") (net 6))
 (segment (start 147 88) (end 148 88) (width 0.2) (layer "F.Cu") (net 6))
 (segment (start 131.58 89.08) (end 128 85.5) (width 0.2) (layer "F.Cu") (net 6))
 (segment (start 128 85.5) (end 128 84.5) (width 0.2) (layer "F.Cu") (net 6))
 (segment (start 131.58 90.5) (end 131.58 89.08) (width 0.2) (layer "F.Cu") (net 6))
 (segment (start 146.5 88.5) (end 147 88) (width 0.2) (layer "F.Cu") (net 6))
 (segment (start 135.5 92) (end 134.5 92) (width 0.2) (layer "F.Cu") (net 6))
 (via (at 148 88) (size 0.6) (drill 0.3) (layers "F.Cu" "B.Cu") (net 6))
 (via (at 134.5 92) (size 0.6) (drill 0.3) (layers "F.Cu" "B.Cu") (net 6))
 (segment (start 149.42 88) (end 150.92 89.5) (width 0.2) (layer "B.Cu") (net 6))
 (segment (start 134.5 92) (end 133.08 92) (width 0.2) (layer "B.Cu") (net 6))
 (segment (start 148 88) (end 149.42 88) (width 0.2) (layer "B.Cu") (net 6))
 (segment (start 133.08 92) (end 131.58 90.5) (width 0.2) (layer "B.Cu") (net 6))
 (segment (start 107.2 90) (end 107.2 87.8) (width 0.2) (layer "F.Cu") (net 1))
 (segment (start 175.3 90) (end 175.3 92.2) (width 0.2) (layer "F.Cu") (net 1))
 (segment (start 123.77 82.27) (end 123.77 84) (width 0.2) (layer "F.Cu") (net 1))
 (segment (start 160 99) (end 158.73 97.73) (width 0.2) (layer "F.Cu") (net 1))
 (segment (start 107.2 87.8) (end 114 81) (width 0.2) (layer "F.Cu") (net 1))
 (segment (start 158.73 97.73) (end 158.73 96) (width 0.2) (layer "F.Cu") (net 1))
 (segment (start 122.5 81) (end 123.77 82.27) (width 0.2) (layer "F.Cu") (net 1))
 (segment (start 114 81) (end 122.5 81) (width 0.2) (layer "F.Cu") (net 1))
 (segment (start 168.5 99) (end 160 99) (width 0.2) (layer "F.Cu") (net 1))
 (segment (start 175.3 92.2) (end 168.5 99) (width 0.2) (layer "F.Cu") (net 1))
 (segment (start 114.8 86.2) (end 118.5 82.5) (width 0.2) (layer "F.Cu") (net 7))
 (segment (start 167.7 90) (end 167.7 93.8) (width 0.2) (layer "F.Cu") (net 7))
 (segment (start 167.7 93.8) (end 164 97.5) (width 0.2) (layer "F.Cu") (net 7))
 (segment (start 114.8 90) (end 114.8 86.2) (width 0.2) (layer "F.Cu") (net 7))
 (via (at 164 97.5) (size 0.6) (drill 0.3) (layers "F.Cu" "B.Cu") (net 7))
 (via (at 118.5 82.5) (size 0.6) (drill 0.3) (layers "F.Cu" "B.Cu") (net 7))
 (segment (start 128.54 82.5) (end 130.54 84.5) (width 0.2) (layer "B.Cu") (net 7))
 (segment (start 153.96 97.5) (end 151.96 95.5) (width 0.2) (layer "B.Cu") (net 7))
 (segment (start 164 97.5) (end 153.96 97.5) (width 0.2) (layer "B.Cu") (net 7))
 (segment (start 118.5 82.5) (end 128.54 82.5) (width 0.2) (layer "B.Cu") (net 7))
 (segment (start 124.2 94.7) (end 124.2 96.5) (width 0.2) (layer "F.Cu") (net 2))
 (segment (start 121.42 90.5) (end 121.42 91.92) (width 0.2) (layer "F.Cu") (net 2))
 (segment (start 122.5 87.5) (end 121.42 88.58) (width 0.2) (layer "F.Cu") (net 2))
 (segment (start 161.08 89.5) (end 161.08 88.08) (width 0.2) (layer "F.Cu") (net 2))
 (segment (start 121.42 91.92) (end 124.2 94.7) (width 0.2) (layer "F.Cu") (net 2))
 (segment (start 161.08 88.08) (end 158.3 85.3) (width 0.2) (layer "F.Cu") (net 2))
 (segment (start 161.08 91.42) (end 161.08 89.5) (width 0.2) (layer "F.Cu") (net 2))
 (segment (start 160 96) (end 160 92.5) (width 0.2) (layer "F.Cu") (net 2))
 (segment (start 121.42 88.58) (end 121.42 90.5) (width 0.2) (layer "F.Cu") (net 2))
 (segment (start 160 92.5) (end 161.08 91.42) (width 0.2) (layer "F.Cu") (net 2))
 (segment (start 122.5 84) (end 122.5 87.5) (width 0.2) (layer "F.Cu") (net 2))
 (segment (start 158.3 85.3) (end 158.3 83.5) (width 0.2) (layer "F.Cu") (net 2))
 (segment (start 161.27 94.23) (end 163.5 92) (width 0.2) (layer "F.Cu") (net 3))
 (segment (start 163.5 92) (end 163.5 85.3) (width 0.2) (layer "F.Cu") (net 3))
 (segment (start 119 88) (end 119 94.7) (width 0.2) (layer "F.Cu") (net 3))
 (segment (start 161.27 96) (end 161.27 94.23) (width 0.2) (layer "F.Cu") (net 3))
 (segment (start 163.5 85.3) (end 161.7 83.5) (width 0.2) (layer "F.Cu") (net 3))
 (segment (start 133.1425 99.5) (end 134.5 98.1425) (width 0.2) (layer "F.Cu") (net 3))
 (segment (start 121.23 84) (end 121.23 85.77) (width 0.2) (layer "F.Cu") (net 3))
 (segment (start 158.7 80.5) (end 149.3575 80.5) (width 0.2) (layer "F.Cu") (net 3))
 (segment (start 161.7 83.5) (end 158.7 80.5) (width 0.2) (layer "F.Cu") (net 3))
 (segment (start 149.3575 80.5) (end 148 81.8575) (width 0.2) (layer "F.Cu") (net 3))
 (segment (start 123.8 99.5) (end 133.1425 99.5) (width 0.2) (layer "F.Cu") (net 3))
 (segment (start 120.8 96.5) (end 123.8 99.5) (width 0.2) (layer "F.Cu") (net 3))
 (segment (start 119 94.7) (end 120.8 96.5) (width 0.2) (layer "F.Cu") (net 3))
 (segment (start 121.23 85.77) (end 119 88) (width 0.2) (layer "F.Cu") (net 3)))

